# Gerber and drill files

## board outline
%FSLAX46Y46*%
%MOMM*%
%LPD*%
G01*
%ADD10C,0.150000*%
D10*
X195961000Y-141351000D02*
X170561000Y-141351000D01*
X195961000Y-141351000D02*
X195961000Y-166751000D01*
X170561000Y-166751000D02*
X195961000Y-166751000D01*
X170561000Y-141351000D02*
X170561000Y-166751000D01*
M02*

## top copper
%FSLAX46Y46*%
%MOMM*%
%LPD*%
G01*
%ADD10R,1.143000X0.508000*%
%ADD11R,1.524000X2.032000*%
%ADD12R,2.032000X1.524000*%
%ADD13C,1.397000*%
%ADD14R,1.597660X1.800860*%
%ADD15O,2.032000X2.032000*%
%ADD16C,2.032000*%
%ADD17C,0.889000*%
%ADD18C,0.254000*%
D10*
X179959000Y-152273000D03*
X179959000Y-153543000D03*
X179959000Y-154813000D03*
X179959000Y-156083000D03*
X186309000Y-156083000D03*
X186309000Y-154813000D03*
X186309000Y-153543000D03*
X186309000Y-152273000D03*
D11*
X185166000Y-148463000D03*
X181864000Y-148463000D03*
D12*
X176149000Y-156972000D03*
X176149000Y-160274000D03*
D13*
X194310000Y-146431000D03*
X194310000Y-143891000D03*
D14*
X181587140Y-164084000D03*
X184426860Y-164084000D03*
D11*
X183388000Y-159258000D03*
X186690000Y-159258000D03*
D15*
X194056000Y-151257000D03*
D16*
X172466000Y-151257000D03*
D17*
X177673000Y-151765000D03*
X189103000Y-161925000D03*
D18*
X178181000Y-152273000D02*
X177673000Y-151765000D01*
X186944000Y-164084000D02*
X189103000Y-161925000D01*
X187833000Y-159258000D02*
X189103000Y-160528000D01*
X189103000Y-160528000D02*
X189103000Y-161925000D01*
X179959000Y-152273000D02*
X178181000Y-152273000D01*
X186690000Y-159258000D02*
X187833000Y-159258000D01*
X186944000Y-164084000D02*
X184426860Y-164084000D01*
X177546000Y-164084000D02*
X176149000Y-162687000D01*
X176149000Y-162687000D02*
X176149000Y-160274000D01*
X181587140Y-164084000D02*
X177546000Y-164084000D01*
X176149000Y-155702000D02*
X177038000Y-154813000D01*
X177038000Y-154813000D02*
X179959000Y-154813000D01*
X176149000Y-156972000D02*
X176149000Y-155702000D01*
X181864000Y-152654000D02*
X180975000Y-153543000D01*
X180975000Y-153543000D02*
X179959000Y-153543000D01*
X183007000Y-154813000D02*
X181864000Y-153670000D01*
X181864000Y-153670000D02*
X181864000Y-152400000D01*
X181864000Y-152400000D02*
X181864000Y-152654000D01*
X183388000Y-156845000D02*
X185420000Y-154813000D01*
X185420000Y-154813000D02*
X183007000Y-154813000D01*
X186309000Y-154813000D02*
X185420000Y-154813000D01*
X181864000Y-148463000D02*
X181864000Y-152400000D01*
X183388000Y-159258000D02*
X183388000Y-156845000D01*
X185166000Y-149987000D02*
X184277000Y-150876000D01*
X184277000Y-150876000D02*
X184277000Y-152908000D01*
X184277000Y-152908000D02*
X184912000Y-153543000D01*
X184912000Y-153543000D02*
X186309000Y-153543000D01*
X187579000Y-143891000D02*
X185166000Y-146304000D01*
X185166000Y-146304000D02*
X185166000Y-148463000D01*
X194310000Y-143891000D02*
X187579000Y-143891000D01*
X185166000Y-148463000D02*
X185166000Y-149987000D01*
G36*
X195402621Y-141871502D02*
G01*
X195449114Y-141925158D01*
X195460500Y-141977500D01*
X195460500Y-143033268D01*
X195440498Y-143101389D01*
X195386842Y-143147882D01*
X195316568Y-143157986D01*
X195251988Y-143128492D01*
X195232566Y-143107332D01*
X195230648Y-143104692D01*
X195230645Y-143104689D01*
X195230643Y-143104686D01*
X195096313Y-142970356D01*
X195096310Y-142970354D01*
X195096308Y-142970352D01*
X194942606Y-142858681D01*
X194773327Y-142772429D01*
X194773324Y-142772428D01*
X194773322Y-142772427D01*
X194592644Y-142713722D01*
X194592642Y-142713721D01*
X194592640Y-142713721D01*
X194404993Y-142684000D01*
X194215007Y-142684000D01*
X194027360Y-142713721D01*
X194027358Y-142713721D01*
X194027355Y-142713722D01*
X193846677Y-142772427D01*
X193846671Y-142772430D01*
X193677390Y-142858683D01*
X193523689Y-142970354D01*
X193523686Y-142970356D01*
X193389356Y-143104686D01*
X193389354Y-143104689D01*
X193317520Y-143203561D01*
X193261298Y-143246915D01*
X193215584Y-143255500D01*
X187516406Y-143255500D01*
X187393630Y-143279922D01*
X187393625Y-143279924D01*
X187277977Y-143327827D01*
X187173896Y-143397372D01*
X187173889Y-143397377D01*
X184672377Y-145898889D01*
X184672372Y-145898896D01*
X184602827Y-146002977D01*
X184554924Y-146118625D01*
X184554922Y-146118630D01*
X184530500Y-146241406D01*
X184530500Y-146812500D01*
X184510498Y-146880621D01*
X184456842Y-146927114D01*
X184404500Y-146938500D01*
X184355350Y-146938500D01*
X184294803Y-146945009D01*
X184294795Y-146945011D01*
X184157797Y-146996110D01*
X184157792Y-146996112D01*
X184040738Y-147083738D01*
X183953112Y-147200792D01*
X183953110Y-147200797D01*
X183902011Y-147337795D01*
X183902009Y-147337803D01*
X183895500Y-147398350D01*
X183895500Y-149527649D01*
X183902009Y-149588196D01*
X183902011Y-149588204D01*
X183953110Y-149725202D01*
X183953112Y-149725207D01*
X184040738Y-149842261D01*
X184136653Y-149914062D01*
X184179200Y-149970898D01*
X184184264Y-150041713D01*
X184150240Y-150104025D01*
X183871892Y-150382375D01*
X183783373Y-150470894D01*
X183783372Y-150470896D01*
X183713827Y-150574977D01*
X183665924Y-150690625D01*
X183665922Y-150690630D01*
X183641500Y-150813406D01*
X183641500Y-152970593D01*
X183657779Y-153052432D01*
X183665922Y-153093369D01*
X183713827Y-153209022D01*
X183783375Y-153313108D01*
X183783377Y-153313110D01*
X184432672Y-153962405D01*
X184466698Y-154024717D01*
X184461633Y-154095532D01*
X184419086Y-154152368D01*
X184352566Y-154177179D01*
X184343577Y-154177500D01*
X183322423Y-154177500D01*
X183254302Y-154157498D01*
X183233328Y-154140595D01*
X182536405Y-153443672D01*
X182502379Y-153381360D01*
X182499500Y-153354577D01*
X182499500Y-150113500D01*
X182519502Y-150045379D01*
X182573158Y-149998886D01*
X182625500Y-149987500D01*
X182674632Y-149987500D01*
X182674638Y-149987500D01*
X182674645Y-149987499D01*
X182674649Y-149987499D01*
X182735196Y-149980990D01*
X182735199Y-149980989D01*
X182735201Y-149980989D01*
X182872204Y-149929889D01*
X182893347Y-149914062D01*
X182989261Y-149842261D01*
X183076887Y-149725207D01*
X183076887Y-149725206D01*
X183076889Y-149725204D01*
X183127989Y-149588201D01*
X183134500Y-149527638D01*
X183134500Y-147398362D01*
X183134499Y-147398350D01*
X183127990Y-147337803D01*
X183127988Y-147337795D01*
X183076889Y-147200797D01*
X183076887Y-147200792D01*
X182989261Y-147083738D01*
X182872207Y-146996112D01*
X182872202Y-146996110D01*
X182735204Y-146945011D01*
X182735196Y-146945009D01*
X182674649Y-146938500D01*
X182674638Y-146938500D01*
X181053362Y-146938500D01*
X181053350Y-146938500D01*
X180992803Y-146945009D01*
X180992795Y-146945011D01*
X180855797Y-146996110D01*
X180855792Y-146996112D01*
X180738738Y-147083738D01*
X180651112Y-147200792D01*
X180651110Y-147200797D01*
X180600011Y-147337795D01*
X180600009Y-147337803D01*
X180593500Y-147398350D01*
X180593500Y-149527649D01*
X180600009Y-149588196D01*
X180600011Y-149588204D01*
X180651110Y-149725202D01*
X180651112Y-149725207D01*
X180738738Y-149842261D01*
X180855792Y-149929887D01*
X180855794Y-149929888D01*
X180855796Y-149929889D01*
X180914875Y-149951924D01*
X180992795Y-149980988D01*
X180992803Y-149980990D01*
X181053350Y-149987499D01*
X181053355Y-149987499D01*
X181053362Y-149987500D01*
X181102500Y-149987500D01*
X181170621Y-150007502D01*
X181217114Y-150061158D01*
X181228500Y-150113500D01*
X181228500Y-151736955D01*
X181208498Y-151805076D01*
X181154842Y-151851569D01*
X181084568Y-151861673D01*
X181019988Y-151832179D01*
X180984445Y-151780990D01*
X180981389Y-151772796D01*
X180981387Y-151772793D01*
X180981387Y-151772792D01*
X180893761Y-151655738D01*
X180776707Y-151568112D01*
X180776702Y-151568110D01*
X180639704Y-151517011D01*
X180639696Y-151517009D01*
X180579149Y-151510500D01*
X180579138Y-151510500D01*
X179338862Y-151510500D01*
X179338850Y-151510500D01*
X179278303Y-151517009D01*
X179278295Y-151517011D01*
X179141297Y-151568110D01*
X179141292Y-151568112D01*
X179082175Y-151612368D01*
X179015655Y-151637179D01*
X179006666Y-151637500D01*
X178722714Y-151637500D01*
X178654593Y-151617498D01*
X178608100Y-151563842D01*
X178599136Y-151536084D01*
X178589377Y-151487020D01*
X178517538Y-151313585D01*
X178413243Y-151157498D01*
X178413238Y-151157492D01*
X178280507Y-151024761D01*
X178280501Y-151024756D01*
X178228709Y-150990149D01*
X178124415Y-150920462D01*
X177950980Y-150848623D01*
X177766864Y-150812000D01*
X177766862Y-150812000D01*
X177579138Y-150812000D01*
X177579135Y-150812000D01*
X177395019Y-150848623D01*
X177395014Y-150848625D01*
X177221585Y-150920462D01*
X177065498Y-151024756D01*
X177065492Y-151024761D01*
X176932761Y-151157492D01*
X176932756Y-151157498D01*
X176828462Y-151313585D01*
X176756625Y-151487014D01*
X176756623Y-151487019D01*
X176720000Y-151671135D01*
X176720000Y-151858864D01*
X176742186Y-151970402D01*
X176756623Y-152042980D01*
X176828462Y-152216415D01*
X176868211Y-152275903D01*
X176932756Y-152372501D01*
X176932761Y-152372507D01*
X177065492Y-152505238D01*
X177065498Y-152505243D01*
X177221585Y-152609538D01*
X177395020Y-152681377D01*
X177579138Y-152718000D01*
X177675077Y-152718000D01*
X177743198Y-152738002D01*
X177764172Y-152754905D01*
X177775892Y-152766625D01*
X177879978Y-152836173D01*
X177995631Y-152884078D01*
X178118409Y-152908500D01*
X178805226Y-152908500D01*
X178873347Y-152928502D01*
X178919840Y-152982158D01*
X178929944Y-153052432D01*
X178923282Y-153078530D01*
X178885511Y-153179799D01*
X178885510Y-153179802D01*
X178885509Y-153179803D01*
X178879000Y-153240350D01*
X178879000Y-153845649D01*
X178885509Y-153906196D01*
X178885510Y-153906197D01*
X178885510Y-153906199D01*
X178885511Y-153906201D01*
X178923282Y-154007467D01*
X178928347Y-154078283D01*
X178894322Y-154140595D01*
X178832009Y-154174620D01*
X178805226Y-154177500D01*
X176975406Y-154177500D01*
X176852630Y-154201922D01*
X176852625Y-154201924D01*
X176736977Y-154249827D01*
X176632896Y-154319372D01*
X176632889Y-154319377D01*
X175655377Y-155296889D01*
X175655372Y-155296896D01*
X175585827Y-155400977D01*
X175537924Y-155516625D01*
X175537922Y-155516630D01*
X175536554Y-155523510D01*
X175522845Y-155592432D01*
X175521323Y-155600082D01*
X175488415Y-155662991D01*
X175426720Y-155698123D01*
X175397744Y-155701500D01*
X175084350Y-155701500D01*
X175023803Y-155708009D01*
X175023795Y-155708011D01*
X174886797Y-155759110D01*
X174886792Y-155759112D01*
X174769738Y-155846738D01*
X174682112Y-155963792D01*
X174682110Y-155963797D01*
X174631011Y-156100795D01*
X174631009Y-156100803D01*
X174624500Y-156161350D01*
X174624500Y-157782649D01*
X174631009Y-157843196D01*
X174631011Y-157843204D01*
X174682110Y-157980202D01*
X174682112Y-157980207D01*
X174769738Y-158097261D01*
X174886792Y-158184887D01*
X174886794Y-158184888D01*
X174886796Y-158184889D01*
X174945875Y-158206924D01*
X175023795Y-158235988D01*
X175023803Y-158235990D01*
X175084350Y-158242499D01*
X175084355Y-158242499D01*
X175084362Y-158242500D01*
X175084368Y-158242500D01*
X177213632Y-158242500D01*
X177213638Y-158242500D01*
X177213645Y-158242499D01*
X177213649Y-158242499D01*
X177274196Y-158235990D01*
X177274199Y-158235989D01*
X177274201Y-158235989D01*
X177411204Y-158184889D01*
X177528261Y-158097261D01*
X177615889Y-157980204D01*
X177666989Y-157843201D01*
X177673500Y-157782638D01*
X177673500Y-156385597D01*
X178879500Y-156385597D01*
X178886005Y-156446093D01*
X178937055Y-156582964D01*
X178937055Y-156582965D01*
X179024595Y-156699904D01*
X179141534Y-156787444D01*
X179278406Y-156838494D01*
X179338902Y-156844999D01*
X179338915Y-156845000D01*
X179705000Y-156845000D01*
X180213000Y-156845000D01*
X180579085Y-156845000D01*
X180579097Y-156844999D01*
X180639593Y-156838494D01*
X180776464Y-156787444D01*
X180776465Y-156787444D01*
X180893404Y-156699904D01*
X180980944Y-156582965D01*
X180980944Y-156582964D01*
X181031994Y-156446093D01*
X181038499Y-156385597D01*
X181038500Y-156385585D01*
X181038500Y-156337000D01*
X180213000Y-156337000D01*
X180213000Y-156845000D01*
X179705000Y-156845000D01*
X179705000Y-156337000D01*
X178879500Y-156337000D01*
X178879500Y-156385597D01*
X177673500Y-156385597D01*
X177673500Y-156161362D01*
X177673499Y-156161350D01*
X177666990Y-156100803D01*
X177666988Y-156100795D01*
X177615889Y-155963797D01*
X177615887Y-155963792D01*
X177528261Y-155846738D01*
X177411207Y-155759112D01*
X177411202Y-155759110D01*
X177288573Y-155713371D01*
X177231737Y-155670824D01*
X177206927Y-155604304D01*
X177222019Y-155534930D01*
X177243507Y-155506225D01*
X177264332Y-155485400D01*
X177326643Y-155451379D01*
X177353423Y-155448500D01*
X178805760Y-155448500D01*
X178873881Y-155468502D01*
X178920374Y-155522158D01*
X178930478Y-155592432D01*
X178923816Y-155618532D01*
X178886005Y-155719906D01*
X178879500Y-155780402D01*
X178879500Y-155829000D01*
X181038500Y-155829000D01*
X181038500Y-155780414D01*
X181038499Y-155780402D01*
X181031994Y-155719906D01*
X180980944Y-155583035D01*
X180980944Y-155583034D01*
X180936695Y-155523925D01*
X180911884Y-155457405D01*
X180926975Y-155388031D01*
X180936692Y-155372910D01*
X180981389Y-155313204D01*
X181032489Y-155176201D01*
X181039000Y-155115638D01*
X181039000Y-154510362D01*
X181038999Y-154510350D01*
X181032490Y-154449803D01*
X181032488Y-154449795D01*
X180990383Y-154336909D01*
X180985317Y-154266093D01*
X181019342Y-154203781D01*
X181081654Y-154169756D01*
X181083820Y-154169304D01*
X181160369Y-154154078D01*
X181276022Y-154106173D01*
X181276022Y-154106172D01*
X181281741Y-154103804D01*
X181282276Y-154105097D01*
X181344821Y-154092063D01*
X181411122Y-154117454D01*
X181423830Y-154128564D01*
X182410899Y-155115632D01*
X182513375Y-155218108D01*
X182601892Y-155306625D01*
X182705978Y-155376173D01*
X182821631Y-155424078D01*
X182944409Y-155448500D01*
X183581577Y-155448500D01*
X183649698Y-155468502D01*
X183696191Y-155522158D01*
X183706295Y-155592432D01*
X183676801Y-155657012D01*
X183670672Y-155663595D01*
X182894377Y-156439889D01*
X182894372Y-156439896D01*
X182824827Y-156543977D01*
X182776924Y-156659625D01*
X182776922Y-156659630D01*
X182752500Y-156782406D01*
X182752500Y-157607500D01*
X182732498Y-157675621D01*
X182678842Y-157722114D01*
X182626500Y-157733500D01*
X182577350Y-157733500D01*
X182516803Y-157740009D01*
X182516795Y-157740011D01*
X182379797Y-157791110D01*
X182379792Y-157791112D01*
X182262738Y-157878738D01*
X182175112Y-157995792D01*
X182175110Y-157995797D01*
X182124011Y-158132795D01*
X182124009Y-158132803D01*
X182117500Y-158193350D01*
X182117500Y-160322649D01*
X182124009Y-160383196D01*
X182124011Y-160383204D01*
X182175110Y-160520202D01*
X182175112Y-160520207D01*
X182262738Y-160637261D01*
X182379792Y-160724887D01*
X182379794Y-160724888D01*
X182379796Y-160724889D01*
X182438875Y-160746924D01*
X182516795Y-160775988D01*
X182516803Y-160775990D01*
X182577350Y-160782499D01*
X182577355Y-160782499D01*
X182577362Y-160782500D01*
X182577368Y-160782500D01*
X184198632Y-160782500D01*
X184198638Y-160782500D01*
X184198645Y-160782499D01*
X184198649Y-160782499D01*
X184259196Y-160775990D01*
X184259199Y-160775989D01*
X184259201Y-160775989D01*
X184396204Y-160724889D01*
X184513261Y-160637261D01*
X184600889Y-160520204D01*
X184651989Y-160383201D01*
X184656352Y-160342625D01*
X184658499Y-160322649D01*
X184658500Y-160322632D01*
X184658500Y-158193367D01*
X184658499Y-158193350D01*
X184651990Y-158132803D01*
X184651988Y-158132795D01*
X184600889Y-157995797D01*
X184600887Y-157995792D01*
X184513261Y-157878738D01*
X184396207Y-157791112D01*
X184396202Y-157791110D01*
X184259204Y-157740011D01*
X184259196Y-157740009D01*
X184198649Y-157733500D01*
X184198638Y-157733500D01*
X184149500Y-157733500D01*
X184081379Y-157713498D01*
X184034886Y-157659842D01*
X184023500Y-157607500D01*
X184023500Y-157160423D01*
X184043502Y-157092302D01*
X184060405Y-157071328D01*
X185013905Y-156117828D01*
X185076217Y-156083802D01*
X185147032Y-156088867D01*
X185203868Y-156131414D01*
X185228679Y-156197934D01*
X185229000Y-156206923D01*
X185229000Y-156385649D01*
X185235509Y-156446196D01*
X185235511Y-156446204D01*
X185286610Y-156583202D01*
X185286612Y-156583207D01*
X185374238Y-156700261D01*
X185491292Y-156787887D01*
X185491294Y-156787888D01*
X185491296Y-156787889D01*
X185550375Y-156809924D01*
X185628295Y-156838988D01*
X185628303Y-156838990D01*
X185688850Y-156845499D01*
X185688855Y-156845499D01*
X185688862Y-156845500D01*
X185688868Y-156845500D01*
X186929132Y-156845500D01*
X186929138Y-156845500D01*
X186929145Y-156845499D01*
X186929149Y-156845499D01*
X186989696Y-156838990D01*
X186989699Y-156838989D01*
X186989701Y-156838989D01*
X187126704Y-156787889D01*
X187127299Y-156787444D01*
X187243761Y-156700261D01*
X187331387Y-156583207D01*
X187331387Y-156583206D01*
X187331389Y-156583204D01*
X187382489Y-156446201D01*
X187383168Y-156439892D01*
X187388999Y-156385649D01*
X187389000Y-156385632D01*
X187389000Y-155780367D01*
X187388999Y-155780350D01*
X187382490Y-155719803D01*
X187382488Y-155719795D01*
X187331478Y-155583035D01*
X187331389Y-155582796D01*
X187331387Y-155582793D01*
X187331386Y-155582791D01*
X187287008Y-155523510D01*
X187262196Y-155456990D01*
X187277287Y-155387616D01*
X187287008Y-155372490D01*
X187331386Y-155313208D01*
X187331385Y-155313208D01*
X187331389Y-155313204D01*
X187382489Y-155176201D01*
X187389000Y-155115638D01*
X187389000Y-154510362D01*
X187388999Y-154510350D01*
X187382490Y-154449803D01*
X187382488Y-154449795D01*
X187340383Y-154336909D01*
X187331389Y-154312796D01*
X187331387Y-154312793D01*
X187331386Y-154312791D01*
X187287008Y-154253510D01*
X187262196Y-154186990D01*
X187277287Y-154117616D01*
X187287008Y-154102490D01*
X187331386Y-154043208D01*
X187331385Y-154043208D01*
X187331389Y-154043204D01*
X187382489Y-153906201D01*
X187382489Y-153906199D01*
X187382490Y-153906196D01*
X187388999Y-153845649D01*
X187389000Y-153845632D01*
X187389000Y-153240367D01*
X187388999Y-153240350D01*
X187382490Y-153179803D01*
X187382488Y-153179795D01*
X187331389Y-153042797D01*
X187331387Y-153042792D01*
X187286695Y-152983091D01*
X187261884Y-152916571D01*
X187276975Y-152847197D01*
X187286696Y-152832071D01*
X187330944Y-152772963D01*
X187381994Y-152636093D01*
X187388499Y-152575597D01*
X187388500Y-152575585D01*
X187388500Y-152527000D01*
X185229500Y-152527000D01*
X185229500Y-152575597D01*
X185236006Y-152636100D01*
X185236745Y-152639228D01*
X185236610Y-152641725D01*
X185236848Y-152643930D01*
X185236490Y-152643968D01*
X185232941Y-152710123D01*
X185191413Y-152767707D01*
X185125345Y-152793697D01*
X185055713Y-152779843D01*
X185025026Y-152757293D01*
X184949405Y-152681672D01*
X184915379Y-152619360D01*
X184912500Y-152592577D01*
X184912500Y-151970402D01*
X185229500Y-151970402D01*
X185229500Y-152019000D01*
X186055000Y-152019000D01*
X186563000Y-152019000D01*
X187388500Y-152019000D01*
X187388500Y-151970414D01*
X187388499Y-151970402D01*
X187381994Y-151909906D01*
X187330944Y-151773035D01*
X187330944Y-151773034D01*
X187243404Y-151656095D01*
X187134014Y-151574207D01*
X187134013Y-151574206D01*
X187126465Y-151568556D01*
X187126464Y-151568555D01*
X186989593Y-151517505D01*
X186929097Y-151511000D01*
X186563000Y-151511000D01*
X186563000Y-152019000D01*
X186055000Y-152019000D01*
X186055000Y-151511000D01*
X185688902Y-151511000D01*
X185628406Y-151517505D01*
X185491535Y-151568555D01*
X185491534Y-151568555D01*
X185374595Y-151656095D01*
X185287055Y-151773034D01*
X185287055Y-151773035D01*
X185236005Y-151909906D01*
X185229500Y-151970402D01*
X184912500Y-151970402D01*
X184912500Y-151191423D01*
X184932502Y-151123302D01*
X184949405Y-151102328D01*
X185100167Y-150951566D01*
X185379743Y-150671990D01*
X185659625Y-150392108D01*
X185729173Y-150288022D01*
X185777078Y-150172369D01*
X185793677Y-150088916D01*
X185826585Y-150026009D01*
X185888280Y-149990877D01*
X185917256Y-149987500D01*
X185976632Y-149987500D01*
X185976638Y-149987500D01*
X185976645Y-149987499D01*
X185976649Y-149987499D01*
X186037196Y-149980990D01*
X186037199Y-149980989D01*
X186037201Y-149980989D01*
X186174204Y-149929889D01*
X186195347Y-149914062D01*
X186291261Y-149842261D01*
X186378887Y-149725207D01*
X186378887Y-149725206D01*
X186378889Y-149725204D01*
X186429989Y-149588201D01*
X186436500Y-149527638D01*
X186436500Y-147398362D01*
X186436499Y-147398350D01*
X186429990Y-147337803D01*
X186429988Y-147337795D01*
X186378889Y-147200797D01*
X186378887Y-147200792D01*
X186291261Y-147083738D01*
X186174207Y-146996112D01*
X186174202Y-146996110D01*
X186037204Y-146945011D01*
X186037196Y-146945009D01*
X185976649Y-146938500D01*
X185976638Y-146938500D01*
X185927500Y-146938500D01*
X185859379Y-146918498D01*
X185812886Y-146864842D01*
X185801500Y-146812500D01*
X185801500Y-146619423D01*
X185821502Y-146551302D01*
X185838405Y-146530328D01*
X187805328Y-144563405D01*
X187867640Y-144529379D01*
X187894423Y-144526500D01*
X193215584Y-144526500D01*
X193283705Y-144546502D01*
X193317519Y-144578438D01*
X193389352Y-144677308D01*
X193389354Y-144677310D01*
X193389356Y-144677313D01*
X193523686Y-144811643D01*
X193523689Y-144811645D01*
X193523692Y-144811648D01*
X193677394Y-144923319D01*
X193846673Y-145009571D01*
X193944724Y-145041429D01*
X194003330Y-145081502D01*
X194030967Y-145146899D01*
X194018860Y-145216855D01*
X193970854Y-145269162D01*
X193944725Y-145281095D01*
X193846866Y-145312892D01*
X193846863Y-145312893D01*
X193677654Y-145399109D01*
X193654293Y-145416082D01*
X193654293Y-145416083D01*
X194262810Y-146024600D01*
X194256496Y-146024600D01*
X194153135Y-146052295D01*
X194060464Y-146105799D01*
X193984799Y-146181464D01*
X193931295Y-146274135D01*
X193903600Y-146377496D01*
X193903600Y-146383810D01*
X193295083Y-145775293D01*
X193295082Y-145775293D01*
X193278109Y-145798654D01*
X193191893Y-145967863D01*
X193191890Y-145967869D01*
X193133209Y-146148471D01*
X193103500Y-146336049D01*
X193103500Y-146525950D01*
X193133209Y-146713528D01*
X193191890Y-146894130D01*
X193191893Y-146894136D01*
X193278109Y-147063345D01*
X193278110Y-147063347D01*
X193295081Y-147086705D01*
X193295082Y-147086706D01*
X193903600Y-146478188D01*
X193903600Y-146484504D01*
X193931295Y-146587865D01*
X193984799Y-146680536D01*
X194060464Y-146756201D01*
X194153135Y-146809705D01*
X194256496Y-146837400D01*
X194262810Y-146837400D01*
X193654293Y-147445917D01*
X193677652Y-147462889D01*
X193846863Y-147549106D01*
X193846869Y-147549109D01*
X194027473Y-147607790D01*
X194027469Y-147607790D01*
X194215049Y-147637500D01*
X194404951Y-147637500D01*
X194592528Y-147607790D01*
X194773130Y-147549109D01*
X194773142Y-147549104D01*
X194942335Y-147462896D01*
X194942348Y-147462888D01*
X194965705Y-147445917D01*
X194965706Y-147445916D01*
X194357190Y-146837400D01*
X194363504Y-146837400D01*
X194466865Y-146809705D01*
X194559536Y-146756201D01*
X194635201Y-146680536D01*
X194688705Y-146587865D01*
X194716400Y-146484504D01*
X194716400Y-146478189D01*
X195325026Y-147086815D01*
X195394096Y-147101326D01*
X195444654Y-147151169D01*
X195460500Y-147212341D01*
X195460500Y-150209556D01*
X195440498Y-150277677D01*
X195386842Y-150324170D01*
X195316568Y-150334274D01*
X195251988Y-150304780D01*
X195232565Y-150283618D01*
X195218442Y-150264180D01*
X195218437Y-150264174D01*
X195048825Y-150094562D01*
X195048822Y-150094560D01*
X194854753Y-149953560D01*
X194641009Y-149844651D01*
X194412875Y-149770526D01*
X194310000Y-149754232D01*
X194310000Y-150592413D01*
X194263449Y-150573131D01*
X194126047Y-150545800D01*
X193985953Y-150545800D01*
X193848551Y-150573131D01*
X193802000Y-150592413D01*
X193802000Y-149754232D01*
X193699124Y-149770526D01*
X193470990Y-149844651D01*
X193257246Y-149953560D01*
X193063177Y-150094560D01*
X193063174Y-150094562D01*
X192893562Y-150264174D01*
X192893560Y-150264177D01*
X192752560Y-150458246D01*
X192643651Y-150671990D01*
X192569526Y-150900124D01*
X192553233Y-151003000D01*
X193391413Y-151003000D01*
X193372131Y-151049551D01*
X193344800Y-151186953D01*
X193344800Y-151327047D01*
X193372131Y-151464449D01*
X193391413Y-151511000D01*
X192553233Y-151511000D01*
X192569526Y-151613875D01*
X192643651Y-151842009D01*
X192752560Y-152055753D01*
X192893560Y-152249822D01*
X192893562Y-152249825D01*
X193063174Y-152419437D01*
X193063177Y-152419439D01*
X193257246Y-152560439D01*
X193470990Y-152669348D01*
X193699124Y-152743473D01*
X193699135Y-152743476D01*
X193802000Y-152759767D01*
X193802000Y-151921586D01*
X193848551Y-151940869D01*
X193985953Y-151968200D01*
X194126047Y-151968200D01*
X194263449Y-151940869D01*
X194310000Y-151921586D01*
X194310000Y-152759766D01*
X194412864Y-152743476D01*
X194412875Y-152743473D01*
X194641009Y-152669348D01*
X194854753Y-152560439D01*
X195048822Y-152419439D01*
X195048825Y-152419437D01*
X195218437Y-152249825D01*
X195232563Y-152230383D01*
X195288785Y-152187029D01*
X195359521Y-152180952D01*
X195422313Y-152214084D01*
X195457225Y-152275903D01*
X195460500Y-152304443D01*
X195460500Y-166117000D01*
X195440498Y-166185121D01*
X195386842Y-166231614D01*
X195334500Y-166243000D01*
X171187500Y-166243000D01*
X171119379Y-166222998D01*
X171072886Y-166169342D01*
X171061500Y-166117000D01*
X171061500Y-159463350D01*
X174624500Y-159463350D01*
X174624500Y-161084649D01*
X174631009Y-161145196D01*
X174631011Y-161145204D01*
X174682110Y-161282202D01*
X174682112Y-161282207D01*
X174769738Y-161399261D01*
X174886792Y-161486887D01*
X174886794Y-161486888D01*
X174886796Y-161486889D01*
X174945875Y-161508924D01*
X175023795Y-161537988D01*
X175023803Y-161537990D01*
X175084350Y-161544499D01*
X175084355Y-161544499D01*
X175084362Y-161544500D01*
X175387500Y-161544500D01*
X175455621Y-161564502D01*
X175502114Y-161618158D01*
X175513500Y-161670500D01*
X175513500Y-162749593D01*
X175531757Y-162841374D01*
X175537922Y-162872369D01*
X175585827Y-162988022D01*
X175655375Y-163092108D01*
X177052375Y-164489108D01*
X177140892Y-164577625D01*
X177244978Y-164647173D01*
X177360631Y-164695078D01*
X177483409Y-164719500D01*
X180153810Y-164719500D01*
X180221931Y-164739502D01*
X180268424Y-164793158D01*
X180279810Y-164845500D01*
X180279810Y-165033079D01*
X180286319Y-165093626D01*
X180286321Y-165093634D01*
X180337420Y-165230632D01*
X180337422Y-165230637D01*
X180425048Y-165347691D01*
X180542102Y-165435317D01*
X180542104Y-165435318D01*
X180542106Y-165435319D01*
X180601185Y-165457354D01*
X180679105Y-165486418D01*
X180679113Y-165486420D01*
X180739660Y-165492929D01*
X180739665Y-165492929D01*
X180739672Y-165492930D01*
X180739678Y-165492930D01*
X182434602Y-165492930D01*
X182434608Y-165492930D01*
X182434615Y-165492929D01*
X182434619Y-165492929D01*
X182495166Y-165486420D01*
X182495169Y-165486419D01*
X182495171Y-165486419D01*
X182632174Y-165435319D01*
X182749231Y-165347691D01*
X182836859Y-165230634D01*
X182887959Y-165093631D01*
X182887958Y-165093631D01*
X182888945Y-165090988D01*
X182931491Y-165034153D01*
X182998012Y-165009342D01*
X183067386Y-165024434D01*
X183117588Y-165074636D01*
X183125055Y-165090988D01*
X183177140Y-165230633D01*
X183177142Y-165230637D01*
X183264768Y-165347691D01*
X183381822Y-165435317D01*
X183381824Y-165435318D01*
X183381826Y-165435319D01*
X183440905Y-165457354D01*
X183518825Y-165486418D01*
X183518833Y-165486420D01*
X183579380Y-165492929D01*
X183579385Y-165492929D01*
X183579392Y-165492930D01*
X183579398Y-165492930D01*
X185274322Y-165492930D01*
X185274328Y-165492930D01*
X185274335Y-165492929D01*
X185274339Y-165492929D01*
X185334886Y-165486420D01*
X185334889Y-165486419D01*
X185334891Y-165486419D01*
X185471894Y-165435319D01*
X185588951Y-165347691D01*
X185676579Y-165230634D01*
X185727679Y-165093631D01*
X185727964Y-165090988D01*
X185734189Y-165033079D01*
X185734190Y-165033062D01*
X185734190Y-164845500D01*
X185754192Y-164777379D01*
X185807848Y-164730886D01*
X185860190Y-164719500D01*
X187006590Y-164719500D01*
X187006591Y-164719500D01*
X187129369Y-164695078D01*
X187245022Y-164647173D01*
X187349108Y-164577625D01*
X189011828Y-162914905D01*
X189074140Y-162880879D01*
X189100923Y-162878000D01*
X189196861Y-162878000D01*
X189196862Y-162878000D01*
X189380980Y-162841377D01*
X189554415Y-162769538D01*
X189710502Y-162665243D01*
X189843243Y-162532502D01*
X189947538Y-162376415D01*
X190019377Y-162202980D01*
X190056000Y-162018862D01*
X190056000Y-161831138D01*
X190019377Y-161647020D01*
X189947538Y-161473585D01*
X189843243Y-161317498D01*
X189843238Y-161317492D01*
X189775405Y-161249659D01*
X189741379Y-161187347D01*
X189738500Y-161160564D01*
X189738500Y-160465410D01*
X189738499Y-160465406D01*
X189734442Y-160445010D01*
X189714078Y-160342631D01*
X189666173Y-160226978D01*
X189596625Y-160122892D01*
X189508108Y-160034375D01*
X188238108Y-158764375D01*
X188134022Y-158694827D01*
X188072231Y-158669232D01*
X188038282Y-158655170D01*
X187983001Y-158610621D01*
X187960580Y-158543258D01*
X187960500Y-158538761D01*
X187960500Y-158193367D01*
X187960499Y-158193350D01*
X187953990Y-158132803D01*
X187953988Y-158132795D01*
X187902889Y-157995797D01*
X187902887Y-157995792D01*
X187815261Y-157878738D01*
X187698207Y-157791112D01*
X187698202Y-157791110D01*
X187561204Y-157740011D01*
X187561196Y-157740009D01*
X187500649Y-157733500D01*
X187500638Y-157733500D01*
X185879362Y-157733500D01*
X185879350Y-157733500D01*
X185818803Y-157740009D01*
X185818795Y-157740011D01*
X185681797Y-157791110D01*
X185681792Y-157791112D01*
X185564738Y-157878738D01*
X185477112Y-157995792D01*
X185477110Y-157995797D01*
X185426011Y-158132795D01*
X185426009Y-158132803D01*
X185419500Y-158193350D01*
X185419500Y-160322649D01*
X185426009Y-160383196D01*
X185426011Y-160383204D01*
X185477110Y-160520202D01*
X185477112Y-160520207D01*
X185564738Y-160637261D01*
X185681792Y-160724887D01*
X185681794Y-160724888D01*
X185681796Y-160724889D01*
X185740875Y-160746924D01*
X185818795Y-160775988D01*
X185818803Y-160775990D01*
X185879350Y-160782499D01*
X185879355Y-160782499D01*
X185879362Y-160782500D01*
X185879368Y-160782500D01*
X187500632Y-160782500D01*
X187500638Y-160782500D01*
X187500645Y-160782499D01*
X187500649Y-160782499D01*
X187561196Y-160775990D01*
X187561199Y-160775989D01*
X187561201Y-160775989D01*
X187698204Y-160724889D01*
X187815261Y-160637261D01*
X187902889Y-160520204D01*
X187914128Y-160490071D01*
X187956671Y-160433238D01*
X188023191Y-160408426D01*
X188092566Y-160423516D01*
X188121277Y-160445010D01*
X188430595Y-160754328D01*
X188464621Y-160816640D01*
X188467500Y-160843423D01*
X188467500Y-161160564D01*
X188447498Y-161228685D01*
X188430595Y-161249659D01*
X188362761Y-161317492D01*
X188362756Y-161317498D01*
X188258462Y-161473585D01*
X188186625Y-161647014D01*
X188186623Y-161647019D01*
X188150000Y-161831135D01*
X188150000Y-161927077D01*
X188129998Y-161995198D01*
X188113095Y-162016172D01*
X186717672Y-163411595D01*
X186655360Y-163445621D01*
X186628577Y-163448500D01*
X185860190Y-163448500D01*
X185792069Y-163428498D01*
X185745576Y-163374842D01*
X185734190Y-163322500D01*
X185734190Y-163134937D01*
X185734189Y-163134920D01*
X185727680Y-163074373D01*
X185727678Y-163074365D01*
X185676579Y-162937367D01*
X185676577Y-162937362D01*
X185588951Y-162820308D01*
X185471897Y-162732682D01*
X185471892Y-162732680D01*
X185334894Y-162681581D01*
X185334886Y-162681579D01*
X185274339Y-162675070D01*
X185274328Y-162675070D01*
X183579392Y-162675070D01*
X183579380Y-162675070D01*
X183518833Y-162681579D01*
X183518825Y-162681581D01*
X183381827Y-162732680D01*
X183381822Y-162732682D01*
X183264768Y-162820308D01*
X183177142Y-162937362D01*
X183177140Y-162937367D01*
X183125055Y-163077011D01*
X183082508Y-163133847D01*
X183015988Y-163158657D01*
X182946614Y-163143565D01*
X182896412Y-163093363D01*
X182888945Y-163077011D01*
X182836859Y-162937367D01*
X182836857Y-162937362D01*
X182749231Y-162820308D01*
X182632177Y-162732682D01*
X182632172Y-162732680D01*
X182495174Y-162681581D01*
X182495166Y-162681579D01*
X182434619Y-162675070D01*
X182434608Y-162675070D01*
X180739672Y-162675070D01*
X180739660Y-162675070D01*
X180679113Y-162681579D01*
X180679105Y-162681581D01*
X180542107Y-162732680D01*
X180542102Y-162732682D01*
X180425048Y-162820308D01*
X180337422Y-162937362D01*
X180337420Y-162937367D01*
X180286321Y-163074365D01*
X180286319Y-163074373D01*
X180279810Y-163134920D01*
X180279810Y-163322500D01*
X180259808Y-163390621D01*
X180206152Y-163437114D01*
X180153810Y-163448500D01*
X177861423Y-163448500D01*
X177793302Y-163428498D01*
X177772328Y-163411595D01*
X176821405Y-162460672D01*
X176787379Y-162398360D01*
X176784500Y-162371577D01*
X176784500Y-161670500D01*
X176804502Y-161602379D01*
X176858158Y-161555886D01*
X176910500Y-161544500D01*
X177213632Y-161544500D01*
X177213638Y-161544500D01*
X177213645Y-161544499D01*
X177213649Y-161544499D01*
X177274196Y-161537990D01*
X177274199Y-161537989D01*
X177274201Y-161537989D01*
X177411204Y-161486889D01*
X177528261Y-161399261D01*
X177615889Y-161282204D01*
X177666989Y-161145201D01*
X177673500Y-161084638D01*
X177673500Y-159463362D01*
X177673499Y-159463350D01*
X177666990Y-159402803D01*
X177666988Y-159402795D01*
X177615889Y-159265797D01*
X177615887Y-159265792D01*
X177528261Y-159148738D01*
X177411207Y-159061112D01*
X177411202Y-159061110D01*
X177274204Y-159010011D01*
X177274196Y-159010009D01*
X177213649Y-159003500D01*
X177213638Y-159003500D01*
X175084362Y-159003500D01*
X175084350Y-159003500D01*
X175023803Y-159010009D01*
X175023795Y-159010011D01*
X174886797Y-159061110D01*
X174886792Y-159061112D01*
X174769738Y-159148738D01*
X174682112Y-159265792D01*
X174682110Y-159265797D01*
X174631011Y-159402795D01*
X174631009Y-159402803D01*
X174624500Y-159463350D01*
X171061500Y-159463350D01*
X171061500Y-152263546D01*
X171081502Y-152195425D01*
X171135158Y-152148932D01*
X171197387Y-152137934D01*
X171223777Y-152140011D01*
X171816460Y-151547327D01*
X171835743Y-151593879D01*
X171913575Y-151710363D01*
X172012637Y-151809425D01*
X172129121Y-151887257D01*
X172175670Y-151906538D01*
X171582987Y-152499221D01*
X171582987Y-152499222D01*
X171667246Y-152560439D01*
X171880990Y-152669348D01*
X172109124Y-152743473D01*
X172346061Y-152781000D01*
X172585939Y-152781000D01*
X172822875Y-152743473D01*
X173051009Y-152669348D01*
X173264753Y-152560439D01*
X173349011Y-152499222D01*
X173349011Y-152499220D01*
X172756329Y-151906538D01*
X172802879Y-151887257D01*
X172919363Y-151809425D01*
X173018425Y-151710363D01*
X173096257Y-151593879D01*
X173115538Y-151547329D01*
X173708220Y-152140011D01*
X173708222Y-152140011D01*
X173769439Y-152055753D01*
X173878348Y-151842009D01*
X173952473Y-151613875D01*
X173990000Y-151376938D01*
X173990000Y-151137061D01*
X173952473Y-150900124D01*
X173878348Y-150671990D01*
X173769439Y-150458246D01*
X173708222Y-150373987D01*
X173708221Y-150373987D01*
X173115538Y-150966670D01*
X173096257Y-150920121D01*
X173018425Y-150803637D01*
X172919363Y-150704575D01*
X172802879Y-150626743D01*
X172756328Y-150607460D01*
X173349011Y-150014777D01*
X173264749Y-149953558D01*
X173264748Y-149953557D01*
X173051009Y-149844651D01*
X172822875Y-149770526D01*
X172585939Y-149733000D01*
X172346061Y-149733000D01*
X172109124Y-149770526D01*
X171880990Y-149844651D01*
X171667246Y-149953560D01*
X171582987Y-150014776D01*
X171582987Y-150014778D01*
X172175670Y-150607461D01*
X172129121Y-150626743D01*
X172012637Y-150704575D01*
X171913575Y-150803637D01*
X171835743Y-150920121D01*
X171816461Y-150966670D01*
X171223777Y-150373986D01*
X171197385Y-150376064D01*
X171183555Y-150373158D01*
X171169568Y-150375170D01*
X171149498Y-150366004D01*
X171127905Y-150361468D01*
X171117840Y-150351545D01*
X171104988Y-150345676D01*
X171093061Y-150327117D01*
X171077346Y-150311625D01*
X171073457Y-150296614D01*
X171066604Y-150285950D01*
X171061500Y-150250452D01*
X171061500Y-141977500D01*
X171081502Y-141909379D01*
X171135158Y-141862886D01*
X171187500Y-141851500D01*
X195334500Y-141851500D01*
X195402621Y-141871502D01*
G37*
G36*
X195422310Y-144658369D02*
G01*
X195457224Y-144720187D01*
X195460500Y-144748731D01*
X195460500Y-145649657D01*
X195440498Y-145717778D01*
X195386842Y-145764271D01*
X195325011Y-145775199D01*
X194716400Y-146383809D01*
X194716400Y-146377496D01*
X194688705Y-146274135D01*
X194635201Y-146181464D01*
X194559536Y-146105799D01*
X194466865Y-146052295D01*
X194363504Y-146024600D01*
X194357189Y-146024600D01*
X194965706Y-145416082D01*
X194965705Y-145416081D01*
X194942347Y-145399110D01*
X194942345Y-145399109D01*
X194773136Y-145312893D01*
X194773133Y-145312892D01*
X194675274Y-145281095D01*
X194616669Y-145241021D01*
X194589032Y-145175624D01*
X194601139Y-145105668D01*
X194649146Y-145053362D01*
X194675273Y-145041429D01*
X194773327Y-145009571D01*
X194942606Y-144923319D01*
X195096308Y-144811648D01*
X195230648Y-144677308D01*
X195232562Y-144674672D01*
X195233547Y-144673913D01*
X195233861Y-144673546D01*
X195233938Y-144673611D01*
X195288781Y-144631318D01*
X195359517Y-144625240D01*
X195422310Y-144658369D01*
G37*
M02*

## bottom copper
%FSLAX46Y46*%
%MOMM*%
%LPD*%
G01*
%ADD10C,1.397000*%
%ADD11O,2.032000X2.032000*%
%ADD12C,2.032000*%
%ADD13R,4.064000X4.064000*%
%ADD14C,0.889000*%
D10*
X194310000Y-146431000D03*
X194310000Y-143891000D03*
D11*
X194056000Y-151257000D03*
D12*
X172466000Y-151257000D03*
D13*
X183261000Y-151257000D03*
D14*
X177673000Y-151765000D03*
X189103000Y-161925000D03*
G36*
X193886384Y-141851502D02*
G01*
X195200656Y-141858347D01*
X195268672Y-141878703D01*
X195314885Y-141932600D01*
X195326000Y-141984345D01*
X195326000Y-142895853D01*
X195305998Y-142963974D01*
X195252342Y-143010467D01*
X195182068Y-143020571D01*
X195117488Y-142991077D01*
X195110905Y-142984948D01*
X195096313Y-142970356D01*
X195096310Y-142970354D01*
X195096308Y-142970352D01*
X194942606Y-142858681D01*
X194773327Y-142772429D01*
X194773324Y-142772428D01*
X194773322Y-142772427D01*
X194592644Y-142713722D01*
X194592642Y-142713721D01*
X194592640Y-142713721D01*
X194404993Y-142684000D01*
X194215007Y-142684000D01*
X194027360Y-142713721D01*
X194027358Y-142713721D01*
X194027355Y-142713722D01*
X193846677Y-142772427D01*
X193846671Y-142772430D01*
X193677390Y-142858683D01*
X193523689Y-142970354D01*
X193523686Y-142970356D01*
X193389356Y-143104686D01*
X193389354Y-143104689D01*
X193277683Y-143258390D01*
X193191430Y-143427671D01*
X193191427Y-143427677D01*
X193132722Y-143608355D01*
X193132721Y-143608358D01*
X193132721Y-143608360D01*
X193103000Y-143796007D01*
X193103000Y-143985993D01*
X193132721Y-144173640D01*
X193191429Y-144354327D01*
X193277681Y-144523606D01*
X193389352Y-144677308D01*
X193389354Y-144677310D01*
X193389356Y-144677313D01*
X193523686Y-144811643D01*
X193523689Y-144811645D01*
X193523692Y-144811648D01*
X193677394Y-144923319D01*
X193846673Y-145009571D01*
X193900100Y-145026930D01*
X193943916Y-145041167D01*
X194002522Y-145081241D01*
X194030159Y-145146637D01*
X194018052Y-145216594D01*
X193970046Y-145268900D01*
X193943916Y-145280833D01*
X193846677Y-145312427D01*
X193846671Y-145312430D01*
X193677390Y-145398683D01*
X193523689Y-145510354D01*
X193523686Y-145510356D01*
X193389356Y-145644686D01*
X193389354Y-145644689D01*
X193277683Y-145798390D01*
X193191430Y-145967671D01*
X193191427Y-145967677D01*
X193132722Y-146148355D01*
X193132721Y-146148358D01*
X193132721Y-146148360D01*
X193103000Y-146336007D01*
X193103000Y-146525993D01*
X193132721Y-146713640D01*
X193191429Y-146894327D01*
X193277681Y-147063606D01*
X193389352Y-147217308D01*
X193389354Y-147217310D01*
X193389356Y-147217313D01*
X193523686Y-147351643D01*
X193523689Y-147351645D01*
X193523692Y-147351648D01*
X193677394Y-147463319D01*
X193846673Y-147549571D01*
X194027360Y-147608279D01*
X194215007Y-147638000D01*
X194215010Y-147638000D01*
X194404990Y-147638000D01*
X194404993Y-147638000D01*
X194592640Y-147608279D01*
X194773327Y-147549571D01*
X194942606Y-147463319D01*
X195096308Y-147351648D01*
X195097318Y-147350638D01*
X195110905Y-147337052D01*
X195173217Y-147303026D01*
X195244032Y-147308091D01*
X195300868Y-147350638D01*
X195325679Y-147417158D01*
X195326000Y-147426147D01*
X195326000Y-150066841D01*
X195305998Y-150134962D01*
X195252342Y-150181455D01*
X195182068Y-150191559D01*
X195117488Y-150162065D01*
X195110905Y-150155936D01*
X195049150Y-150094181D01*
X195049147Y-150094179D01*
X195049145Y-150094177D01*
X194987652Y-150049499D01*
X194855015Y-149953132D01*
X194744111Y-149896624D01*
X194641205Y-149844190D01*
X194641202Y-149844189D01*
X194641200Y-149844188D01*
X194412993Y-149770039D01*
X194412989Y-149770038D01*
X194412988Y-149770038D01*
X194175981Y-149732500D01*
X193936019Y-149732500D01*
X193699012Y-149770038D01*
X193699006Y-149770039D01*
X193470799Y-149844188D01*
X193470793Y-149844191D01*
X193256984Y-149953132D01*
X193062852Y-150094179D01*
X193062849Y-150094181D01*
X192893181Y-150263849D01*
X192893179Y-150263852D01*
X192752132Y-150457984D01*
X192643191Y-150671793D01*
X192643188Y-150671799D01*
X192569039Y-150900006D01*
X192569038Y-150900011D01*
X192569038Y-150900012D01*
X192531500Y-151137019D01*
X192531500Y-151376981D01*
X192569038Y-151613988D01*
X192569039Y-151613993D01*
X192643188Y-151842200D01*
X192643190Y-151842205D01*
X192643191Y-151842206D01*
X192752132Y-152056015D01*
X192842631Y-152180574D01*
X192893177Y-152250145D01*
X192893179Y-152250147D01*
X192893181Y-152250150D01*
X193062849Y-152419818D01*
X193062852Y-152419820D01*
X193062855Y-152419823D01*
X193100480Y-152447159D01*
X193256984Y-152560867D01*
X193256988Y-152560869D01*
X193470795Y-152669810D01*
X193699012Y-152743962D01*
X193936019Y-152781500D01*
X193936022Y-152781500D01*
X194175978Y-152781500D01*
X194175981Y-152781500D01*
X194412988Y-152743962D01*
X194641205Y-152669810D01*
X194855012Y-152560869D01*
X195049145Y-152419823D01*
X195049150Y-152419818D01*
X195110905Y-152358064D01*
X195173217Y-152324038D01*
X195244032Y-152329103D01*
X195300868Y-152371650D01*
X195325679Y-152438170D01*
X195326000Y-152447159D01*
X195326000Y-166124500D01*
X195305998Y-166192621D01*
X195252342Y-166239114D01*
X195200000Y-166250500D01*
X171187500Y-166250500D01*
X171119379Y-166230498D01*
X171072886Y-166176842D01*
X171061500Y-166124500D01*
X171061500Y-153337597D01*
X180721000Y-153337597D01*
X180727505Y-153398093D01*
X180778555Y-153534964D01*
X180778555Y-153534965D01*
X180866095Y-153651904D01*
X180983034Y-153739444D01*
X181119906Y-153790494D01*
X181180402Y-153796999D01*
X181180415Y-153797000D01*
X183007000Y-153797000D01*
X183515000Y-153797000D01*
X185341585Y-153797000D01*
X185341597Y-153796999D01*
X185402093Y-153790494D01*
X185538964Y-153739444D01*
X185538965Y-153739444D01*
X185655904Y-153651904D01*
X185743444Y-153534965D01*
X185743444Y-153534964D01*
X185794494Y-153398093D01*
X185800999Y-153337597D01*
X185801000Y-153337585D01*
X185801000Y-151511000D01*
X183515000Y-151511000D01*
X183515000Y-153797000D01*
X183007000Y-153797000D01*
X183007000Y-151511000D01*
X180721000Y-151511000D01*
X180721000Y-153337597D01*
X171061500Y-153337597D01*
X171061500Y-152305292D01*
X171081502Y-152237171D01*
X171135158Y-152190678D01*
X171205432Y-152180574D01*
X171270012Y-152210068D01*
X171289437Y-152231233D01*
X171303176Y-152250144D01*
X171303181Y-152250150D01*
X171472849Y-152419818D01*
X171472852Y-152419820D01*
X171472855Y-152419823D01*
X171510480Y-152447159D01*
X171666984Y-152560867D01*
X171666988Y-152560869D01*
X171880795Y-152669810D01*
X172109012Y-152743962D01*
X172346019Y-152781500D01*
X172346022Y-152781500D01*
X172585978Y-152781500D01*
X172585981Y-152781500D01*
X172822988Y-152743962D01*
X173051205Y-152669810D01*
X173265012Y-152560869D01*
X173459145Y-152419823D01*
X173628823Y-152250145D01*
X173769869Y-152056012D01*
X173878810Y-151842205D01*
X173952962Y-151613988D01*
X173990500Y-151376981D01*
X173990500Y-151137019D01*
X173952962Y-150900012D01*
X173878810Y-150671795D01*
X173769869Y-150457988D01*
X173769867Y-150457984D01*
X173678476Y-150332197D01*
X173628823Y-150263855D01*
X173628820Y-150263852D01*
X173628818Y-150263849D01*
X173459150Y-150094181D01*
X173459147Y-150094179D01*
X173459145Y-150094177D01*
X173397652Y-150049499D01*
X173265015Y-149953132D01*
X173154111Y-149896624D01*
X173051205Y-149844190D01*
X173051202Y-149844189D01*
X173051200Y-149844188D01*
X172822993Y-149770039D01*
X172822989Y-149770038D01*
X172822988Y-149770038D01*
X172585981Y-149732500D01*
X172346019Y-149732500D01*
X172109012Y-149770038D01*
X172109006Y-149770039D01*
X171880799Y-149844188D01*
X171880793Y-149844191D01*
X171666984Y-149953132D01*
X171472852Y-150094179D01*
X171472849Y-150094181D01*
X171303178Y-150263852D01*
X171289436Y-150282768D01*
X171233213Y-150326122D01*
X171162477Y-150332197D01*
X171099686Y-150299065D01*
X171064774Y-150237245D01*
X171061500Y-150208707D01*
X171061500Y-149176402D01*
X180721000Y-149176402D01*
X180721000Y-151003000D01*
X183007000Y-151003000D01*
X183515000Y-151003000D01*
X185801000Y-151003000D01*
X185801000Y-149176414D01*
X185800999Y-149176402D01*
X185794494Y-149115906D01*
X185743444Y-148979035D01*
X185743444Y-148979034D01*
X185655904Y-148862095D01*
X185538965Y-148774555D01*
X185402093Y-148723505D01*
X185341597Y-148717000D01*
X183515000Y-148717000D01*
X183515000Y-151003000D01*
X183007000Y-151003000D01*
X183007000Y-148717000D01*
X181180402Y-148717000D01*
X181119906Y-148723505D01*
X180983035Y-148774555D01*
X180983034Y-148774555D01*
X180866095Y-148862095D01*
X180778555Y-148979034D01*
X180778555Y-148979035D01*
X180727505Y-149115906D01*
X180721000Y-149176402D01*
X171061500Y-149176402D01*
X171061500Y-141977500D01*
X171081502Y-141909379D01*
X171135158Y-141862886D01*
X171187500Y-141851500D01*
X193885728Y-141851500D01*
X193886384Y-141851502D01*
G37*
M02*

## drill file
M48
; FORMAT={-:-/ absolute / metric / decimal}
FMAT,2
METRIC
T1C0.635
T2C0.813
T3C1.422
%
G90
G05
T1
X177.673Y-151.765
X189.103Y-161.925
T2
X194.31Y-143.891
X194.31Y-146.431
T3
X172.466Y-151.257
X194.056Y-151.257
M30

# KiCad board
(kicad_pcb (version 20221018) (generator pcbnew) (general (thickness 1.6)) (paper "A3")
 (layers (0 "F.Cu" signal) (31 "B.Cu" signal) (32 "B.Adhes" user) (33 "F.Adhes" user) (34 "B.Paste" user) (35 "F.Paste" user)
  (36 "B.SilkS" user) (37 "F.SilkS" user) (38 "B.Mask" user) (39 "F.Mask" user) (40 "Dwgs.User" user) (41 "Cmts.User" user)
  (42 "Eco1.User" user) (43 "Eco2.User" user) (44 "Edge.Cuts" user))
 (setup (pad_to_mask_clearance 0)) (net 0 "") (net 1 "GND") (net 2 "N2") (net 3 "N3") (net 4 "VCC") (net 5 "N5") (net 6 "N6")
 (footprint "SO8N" (layer "F.Cu") (at 183.134 154.178 -90)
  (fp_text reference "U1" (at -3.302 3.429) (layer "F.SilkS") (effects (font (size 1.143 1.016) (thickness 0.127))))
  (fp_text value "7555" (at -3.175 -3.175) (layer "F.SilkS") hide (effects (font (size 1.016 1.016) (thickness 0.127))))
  (pad "1" smd rect (at -1.905 3.175 270) (size 0.508 1.143) (layers "F.Cu" "F.Paste" "F.Mask") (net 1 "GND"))
  (pad "2" smd rect (at -0.635 3.175 270) (size 0.508 1.143) (layers "F.Cu" "F.Paste" "F.Mask") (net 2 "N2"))
  (pad "3" smd rect (at 0.635 3.175 270) (size 0.508 1.143) (layers "F.Cu" "F.Paste" "F.Mask") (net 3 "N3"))
  (pad "4" smd rect (at 1.905 3.175 270) (size 0.508 1.143) (layers "F.Cu" "F.Paste" "F.Mask") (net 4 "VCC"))
  (pad "5" smd rect (at 1.905 -3.175 270) (size 0.508 1.143) (layers "F.Cu" "F.Paste" "F.Mask"))
  (pad "6" smd rect (at 0.635 -3.175 270) (size 0.508 1.143) (layers "F.Cu" "F.Paste" "F.Mask") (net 2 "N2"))
  (pad "7" smd rect (at -0.635 -3.175 270) (size 0.508 1.143) (layers "F.Cu" "F.Paste" "F.Mask") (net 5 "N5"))
  (pad "8" smd rect (at -1.905 -3.175 270) (size 0.508 1.143) (layers "F.Cu" "F.Paste" "F.Mask") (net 4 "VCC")))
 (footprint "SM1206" (layer "F.Cu") (at 183.515 148.463 180)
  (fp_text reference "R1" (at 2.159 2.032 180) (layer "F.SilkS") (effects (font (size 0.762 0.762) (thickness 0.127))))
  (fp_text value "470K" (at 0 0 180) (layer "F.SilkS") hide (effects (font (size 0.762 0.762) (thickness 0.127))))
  (pad "1" smd rect (at -1.651 0 180) (size 1.524 2.032) (layers "F.Cu" "F.Paste" "F.Mask") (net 5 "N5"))
  (pad "2" smd rect (at 1.651 0 180) (size 1.524 2.032) (layers "F.Cu" "F.Paste" "F.Mask") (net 2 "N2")))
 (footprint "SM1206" (layer "F.Cu") (at 176.149 158.623 -90)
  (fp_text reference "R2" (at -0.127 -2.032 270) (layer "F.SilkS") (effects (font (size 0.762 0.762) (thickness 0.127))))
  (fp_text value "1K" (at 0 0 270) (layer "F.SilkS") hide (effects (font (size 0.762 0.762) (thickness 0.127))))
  (pad "1" smd rect (at -1.651 0 270) (size 1.524 2.032) (layers "F.Cu" "F.Paste" "F.Mask") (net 3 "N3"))
  (pad "2" smd rect (at 1.651 0 270) (size 1.524 2.032) (layers "F.Cu" "F.Paste" "F.Mask") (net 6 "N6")))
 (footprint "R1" (layer "F.Cu") (at 194.31 145.161 90)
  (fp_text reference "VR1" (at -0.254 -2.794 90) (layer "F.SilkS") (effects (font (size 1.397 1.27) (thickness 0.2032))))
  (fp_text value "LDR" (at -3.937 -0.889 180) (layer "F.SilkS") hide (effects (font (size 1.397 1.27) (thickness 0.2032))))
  (pad "1" thru_hole circle (at -1.27 0 90) (size 1.397 1.397) (drill 0.812799) (layers "*.Cu" "*.Mask" "F.SilkS") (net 4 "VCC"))
  (pad "2" thru_hole circle (at 1.27 0 90) (size 1.397 1.397) (drill 0.812799) (layers "*.Cu" "*.Mask" "F.SilkS") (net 5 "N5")))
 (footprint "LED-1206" (layer "F.Cu") (at 183.007 164.084)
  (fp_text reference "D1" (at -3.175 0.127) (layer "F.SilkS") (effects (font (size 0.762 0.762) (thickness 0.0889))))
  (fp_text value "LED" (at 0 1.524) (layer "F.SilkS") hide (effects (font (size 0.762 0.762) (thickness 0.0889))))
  (pad "1" smd rect (at -1.41986 0) (size 1.59766 1.80086) (layers "F.Cu" "F.Paste" "F.Mask") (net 6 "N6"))
  (pad "2" smd rect (at 1.41986 0) (size 1.59766 1.80086) (layers "F.Cu" "F.Paste" "F.Mask") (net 1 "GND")))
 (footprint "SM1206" (layer "F.Cu") (at 185.039 159.258)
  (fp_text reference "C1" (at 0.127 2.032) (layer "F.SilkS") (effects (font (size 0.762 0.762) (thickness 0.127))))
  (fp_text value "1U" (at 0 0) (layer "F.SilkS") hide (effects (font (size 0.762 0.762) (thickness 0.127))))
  (pad "1" smd rect (at -1.651 0) (size 1.524 2.032) (layers "F.Cu" "F.Paste" "F.Mask") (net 2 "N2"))
  (pad "2" smd rect (at 1.651 0) (size 1.524 2.032) (layers "F.Cu" "F.Paste" "F.Mask") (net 1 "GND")))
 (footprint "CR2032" (layer "B.Cu") (at 183.261 151.257 180)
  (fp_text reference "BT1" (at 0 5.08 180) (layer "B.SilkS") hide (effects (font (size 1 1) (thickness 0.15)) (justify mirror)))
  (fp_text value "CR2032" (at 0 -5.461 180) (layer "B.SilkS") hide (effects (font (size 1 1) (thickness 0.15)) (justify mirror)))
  (pad "1" thru_hole oval (at -10.795 0 180) (size 2.032 2.032) (drill 1.4224) (layers "*.Cu" "*.Mask" "B.SilkS") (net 4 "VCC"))
  (pad "1" thru_hole circle (at 10.795 0 180) (size 2.032 2.032) (drill 1.4224) (layers "*.Cu" "*.Mask" "B.SilkS") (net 4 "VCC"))
  (pad "2" smd rect (at 0 0 180) (size 4.064 4.064) (layers "B.Cu" "B.Paste" "B.Mask") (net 1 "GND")))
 (gr_line (start 195.961 141.351) (end 170.561 141.351) (stroke (width 0.15) (type solid)) (layer "Edge.Cuts"))
 (gr_line (start 195.961 141.351) (end 195.961 166.751) (stroke (width 0.15) (type solid)) (layer "Edge.Cuts"))
 (gr_line (start 170.561 166.751) (end 195.961 166.751) (stroke (width 0.15) (type solid)) (layer "Edge.Cuts"))
 (gr_line (start 170.561 141.351) (end 170.561 166.751) (stroke (width 0.15) (type solid)) (layer "Edge.Cuts"))
 (segment (start 178.181 152.273) (end 177.673 151.765) (width 0.254) (layer "F.Cu") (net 1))
 (segment (start 186.944 164.084) (end 189.103 161.925) (width 0.254) (layer "F.Cu") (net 1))
 (segment (start 187.833 159.258) (end 189.103 160.528) (width 0.254) (layer "F.Cu") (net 1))
 (segment (start 189.103 160.528) (end 189.103 161.925) (width 0.254) (layer "F.Cu") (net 1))
 (segment (start 179.959 152.273) (end 178.181 152.273) (width 0.254) (layer "F.Cu") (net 1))
 (segment (start 186.69 159.258) (end 187.833 159.258) (width 0.254) (layer "F.Cu") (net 1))
 (segment (start 186.944 164.084) (end 184.42686 164.084) (width 0.254) (layer "F.Cu") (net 1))
 (via (at 177.673 151.765) (size 0.889) (drill 0.635) (layers "F.Cu" "B.Cu") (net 1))
 (via (at 189.103 161.925) (size 0.889) (drill 0.635) (layers "F.Cu" "B.Cu") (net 1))
 (segment (start 177.546 164.084) (end 176.149 162.687) (width 0.254) (layer "F.Cu") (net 6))
 (segment (start 176.149 162.687) (end 176.149 160.274) (width 0.254) (layer "F.Cu") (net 6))
 (segment (start 181.58714 164.084) (end 177.546 164.084) (width 0.254) (layer "F.Cu") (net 6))
 (segment (start 176.149 155.702) (end 177.038 154.813) (width 0.254) (layer "F.Cu") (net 3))
 (segment (start 177.038 154.813) (end 179.959 154.813) (width 0.254) (layer "F.Cu") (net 3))
 (segment (start 176.149 156.972) (end 176.149 155.702) (width 0.254) (layer "F.Cu") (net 3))
 (segment (start 181.864 152.654) (end 180.975 153.543) (width 0.254) (layer "F.Cu") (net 2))
 (segment (start 180.975 153.543) (end 179.959 153.543) (width 0.254) (layer "F.Cu") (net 2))
 (segment (start 183.007 154.813) (end 181.864 153.67) (width 0.254) (layer "F.Cu") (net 2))
 (segment (start 181.864 153.67) (end 181.864 152.4) (width 0.254) (layer "F.Cu") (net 2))
 (segment (start 181.864 152.4) (end 181.864 152.654) (width 0.254) (layer "F.Cu") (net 2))
 (segment (start 183.388 156.845) (end 185.42 154.813) (width 0.254) (layer "F.Cu") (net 2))
 (segment (start 185.42 154.813) (end 183.007 154.813) (width 0.254) (layer "F.Cu") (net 2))
 (segment (start 186.309 154.813) (end 185.42 154.813) (width 0.254) (layer "F.Cu") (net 2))
 (segment (start 181.864 148.463) (end 181.864 152.4) (width 0.254) (layer "F.Cu") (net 2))
 (segment (start 183.388 159.258) (end 183.388 156.845) (width 0.254) (layer "F.Cu") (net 2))
 (segment (start 185.166 149.987) (end 184.277 150.876) (width 0.254) (layer "F.Cu") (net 5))
 (segment (start 184.277 150.876) (end 184.277 152.908) (width 0.254) (layer "F.Cu") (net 5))
 (segment (start 184.277 152.908) (end 184.912 153.543) (width 0.254) (layer "F.Cu") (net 5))
 (segment (start 184.912 153.543) (end 186.309 153.543) (width 0.254) (layer "F.Cu") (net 5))
 (segment (start 187.579 143.891) (end 185.166 146.304) (width 0.254) (layer "F.Cu") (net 5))
 (segment (start 185.166 146.304) (end 185.166 148.463) (width 0.254) (layer "F.Cu") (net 5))
 (segment (start 194.31 143.891) (end 187.579 143.891) (width 0.254) (layer "F.Cu") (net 5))
 (segment (start 185.166 148.463) (end 185.166 149.987) (width 0.254) (layer "F.Cu") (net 5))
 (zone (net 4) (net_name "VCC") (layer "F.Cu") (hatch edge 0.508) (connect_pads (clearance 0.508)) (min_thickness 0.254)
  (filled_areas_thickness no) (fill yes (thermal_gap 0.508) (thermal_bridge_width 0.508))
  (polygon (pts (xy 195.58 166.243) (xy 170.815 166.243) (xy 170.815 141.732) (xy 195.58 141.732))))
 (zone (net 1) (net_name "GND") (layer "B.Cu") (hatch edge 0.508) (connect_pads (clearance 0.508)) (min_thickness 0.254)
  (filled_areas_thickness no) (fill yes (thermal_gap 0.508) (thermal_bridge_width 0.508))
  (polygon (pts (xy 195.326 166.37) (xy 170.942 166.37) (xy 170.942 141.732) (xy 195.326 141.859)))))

